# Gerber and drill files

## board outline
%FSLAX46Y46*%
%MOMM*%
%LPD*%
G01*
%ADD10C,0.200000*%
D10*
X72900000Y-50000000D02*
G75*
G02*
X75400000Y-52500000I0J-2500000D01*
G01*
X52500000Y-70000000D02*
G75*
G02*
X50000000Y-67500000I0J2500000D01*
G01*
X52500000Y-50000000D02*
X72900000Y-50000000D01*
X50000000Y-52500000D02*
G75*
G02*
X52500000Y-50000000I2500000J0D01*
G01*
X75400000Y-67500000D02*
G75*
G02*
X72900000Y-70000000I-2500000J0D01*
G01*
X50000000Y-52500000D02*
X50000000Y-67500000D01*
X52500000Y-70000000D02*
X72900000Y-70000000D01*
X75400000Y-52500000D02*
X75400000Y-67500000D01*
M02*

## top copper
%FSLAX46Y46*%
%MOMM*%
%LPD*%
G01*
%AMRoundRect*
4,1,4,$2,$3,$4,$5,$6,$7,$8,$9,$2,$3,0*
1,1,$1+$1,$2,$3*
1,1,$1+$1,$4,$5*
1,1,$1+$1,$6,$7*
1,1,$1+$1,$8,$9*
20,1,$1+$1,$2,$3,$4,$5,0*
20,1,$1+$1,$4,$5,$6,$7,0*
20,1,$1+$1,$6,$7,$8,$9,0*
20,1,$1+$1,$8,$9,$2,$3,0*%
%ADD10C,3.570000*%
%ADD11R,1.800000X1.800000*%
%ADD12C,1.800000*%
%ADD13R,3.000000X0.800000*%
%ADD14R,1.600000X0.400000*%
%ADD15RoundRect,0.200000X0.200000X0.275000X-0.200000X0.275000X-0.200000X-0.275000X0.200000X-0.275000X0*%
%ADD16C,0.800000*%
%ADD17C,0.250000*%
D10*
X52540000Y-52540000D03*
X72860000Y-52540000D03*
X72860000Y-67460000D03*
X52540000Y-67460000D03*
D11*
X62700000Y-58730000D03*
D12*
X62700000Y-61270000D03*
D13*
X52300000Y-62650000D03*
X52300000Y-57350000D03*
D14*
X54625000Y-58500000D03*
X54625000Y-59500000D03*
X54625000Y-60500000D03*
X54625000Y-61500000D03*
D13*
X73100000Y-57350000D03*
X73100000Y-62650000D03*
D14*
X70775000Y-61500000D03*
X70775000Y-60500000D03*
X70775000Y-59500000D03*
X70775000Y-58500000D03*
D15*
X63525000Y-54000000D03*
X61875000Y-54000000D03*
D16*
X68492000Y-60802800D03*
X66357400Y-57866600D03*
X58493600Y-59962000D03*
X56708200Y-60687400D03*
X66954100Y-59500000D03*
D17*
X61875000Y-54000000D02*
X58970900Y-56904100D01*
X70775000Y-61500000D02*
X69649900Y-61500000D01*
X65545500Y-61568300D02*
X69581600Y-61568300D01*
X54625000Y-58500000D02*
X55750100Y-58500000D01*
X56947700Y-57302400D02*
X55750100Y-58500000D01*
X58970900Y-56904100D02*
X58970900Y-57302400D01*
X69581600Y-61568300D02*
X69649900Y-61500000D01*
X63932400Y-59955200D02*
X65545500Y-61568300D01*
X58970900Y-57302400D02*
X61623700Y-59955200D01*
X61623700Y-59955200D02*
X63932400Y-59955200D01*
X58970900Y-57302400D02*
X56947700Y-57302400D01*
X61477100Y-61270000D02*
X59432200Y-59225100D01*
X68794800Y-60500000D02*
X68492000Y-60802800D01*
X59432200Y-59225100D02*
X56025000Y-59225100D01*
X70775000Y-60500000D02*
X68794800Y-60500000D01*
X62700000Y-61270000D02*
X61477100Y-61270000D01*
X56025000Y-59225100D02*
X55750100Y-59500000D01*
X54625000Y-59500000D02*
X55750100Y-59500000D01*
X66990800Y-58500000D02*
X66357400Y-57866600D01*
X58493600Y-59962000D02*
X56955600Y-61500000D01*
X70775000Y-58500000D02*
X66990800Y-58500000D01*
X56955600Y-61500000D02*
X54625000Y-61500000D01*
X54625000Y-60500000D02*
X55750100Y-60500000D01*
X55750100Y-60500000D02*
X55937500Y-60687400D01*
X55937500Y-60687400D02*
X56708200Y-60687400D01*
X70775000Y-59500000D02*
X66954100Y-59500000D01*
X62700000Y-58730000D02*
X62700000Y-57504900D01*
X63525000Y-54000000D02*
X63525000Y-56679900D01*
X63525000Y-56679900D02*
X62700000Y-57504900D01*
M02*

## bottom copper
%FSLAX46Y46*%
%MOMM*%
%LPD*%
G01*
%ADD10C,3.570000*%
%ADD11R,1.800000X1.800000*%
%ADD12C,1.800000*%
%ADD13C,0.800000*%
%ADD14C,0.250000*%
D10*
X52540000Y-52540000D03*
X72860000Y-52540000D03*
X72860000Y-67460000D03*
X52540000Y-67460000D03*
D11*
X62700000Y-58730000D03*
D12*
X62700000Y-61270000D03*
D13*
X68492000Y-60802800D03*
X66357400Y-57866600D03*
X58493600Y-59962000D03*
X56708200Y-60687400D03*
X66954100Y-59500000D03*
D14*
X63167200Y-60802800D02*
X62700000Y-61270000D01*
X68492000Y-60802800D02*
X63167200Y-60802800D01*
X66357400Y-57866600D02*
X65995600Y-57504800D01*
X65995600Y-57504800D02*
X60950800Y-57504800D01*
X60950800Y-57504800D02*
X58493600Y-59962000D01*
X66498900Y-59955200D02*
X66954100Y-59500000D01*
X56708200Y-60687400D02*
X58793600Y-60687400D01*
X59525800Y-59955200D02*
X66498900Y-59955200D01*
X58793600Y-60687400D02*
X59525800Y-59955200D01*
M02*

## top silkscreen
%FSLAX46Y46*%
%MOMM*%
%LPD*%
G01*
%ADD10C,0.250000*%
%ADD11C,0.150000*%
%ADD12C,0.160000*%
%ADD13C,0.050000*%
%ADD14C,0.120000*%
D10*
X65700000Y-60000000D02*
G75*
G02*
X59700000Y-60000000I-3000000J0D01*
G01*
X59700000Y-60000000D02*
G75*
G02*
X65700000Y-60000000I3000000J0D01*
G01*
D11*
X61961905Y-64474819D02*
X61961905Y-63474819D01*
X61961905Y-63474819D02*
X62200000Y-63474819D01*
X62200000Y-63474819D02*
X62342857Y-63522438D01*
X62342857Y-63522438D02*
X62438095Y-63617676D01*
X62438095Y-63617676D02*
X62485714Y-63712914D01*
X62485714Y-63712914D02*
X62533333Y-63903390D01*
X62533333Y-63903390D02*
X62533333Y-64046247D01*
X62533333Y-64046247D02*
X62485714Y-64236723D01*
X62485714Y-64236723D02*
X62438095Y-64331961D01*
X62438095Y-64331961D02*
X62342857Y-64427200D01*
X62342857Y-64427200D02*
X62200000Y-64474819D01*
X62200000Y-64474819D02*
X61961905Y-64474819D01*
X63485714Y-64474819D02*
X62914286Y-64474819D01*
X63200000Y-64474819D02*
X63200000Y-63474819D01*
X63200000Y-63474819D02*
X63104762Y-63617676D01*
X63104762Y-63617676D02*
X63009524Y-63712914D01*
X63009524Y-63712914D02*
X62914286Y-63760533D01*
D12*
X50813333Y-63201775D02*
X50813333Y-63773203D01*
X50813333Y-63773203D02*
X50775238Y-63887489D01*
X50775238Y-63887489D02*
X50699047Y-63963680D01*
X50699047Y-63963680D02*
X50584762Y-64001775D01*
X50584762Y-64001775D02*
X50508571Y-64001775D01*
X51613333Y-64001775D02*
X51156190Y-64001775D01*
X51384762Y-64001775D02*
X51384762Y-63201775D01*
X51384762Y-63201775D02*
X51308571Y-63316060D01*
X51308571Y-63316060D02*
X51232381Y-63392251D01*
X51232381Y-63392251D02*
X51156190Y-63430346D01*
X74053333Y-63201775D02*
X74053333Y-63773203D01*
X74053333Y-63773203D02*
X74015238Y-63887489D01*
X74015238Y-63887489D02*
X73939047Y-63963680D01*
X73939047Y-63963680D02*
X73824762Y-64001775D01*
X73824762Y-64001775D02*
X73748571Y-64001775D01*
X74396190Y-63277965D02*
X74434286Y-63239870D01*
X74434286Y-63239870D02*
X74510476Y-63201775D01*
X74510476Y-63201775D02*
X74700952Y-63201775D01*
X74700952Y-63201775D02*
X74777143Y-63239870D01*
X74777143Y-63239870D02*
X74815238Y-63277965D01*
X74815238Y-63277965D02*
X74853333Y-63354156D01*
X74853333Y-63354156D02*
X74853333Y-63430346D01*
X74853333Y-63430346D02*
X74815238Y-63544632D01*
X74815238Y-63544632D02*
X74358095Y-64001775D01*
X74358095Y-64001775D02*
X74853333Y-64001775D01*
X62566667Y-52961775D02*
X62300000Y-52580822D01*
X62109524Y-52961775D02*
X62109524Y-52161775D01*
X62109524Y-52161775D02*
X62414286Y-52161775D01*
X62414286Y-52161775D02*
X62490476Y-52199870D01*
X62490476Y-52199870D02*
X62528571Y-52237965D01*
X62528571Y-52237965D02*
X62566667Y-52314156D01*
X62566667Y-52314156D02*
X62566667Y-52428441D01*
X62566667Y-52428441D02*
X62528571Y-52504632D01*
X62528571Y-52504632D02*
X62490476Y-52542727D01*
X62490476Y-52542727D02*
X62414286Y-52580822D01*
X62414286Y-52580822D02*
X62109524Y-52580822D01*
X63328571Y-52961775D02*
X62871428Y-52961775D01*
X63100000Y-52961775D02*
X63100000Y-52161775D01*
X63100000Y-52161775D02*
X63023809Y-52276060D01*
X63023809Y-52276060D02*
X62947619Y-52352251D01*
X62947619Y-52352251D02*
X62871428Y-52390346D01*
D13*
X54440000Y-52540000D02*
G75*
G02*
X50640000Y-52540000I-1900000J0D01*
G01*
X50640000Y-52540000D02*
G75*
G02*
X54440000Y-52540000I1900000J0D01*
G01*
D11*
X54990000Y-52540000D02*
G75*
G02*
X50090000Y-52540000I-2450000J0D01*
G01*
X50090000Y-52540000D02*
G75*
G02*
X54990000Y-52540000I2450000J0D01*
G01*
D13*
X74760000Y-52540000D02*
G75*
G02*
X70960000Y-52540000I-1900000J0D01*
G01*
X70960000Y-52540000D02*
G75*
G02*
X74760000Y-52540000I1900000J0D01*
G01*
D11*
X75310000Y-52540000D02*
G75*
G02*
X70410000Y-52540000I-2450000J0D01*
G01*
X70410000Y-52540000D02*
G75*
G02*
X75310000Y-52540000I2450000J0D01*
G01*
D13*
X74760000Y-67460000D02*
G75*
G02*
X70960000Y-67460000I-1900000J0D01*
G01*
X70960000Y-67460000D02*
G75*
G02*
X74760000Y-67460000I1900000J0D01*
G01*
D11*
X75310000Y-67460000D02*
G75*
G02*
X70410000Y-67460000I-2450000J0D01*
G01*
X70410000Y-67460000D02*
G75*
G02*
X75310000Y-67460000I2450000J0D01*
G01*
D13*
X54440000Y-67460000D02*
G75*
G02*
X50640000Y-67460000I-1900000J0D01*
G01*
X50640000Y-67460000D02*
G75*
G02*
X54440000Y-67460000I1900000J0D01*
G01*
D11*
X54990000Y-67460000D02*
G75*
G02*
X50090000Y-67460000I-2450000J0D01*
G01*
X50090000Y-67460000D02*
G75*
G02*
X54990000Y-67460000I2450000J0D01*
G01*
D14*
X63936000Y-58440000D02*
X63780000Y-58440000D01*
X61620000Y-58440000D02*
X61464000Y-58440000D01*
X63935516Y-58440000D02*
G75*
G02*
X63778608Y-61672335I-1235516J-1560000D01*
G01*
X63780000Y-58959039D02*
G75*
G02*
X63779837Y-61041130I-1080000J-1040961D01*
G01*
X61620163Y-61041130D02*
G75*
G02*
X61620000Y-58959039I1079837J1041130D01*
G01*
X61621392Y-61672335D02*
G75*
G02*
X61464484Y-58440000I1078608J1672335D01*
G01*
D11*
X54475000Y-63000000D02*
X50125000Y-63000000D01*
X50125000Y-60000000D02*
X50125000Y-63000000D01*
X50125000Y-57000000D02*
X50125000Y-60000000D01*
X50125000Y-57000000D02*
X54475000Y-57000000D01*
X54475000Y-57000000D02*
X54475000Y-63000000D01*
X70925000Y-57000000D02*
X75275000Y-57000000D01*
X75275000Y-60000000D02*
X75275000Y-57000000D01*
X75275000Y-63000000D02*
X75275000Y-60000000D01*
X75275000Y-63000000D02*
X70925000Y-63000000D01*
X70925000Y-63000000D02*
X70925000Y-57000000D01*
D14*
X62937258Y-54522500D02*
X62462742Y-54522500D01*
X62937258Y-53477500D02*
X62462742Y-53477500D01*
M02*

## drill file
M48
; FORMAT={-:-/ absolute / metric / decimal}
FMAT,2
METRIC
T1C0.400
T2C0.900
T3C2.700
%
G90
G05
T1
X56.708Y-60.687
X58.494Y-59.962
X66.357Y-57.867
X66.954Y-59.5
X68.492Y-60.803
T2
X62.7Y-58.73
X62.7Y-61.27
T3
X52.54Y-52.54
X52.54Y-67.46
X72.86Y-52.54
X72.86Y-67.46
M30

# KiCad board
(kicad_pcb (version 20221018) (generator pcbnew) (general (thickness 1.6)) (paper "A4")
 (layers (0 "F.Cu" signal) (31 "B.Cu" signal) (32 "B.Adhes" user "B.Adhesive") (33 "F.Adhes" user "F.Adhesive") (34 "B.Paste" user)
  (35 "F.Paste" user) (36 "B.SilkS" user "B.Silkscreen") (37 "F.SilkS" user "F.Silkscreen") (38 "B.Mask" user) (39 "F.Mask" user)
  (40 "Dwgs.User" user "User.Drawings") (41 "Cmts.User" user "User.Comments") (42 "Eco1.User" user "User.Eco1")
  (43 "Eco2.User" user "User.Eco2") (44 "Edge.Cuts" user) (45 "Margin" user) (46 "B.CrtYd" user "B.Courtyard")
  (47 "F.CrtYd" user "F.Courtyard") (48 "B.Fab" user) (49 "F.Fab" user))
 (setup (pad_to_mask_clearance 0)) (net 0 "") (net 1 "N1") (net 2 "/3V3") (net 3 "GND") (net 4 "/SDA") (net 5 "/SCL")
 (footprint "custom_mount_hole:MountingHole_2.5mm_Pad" (layer "F.Cu") (at 52.54 52.54)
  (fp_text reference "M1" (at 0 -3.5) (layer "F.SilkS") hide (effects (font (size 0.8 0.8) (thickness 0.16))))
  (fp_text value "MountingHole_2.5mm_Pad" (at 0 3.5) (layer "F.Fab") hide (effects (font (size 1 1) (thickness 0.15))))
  (fp_circle (center 0 0) (end 1.9 0) (stroke (width 0.05) (type solid)) (fill none) (layer "F.SilkS"))
  (fp_circle (center 0 0) (end 2.45 0) (stroke (width 0.15) (type solid)) (fill none) (layer "F.SilkS"))
  (pad "~" thru_hole circle (at 0 0) (size 3.57 3.57) (drill 2.7) (layers "*.Cu" "*.Mask")))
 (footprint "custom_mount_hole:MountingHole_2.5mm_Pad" (layer "F.Cu") (at 72.86 52.54)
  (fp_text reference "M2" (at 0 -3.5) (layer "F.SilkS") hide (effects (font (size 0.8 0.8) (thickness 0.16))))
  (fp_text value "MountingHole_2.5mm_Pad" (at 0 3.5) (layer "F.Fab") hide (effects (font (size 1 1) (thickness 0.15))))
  (fp_circle (center 0 0) (end 1.9 0) (stroke (width 0.05) (type solid)) (fill none) (layer "F.SilkS"))
  (fp_circle (center 0 0) (end 2.45 0) (stroke (width 0.15) (type solid)) (fill none) (layer "F.SilkS"))
  (pad "~" thru_hole circle (at 0 0) (size 3.57 3.57) (drill 2.7) (layers "*.Cu" "*.Mask")))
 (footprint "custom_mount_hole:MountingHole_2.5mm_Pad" (layer "F.Cu") (at 72.86 67.46)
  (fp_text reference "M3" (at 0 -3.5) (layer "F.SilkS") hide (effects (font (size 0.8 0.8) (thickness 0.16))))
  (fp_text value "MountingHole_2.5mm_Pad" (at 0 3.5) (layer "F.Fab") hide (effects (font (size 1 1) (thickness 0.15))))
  (fp_circle (center 0 0) (end 1.9 0) (stroke (width 0.05) (type solid)) (fill none) (layer "F.SilkS"))
  (fp_circle (center 0 0) (end 2.45 0) (stroke (width 0.15) (type solid)) (fill none) (layer "F.SilkS"))
  (pad "~" thru_hole circle (at 0 0) (size 3.57 3.57) (drill 2.7) (layers "*.Cu" "*.Mask")))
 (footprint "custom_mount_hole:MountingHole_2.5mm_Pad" (layer "F.Cu") (at 52.54 67.46)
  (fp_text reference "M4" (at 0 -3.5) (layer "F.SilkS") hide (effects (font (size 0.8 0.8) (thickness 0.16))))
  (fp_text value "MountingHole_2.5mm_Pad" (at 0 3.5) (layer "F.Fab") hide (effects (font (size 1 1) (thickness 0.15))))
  (fp_circle (center 0 0) (end 1.9 0) (stroke (width 0.05) (type solid)) (fill none) (layer "F.SilkS"))
  (fp_circle (center 0 0) (end 2.45 0) (stroke (width 0.15) (type solid)) (fill none) (layer "F.SilkS"))
  (pad "~" thru_hole circle (at 0 0) (size 3.57 3.57) (drill 2.7) (layers "*.Cu" "*.Mask")))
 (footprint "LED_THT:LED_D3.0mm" (layer "F.Cu") (at 62.7 58.73 -90)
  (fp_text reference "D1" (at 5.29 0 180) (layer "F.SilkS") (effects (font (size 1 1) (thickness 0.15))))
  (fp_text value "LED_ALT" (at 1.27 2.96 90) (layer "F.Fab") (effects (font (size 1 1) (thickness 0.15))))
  (fp_line (start -0.29 -1.236) (end -0.29 -1.08) (stroke (width 0.12) (type solid)) (layer "F.SilkS"))
  (fp_line (start -0.29 1.08) (end -0.29 1.236) (stroke (width 0.12) (type solid)) (layer "F.SilkS"))
  (fp_arc (start -0.29 -1.235516) (mid 1.366487 -1.987659) (end 2.942335 -1.078608) (stroke (width 0.12) (type solid)) (layer "F.SilkS"))
  (fp_arc (start 0.229039 -1.08) (mid 1.270117 -1.5) (end 2.31113 -1.079837) (stroke (width 0.12) (type solid)) (layer "F.SilkS"))
  (fp_arc (start 2.31113 1.079837) (mid 1.270117 1.5) (end 0.229039 1.08) (stroke (width 0.12) (type solid)) (layer "F.SilkS"))
  (fp_arc (start 2.942335 1.078608) (mid 1.366487 1.987659) (end -0.29 1.235516) (stroke (width 0.12) (type solid)) (layer "F.SilkS"))
  (pad "1" thru_hole rect (at 0 0 270) (size 1.8 1.8) (drill 0.9) (layers "*.Cu" "*.Mask") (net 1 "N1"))
  (pad "2" thru_hole circle (at 2.54 0 270) (size 1.8 1.8) (drill 0.9) (layers "*.Cu" "*.Mask") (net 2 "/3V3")))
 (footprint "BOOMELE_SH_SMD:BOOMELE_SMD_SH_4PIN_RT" (layer "F.Cu") (at 52.78 60 90)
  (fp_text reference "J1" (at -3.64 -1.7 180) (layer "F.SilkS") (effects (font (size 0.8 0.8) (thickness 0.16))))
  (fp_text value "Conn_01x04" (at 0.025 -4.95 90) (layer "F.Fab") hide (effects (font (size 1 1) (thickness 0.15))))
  (fp_line (start -3 1.695) (end -3 -2.655) (stroke (width 0.15) (type solid)) (layer "F.SilkS"))
  (fp_line (start 0 -2.655) (end -3 -2.655) (stroke (width 0.15) (type solid)) (layer "F.SilkS"))
  (fp_line (start 3 -2.655) (end 0 -2.655) (stroke (width 0.15) (type solid)) (layer "F.SilkS"))
  (fp_line (start 3 -2.655) (end 3 1.695) (stroke (width 0.15) (type solid)) (layer "F.SilkS"))
  (fp_line (start 3 1.695) (end -3 1.695) (stroke (width 0.15) (type solid)) (layer "F.SilkS"))
  (pad "" smd rect (at -2.65 -0.48 270) (size 0.8 3) (layers "F.Cu" "F.Paste" "F.Mask"))
  (pad "" smd rect (at 2.65 -0.48 270) (size 0.8 3) (layers "F.Cu" "F.Paste" "F.Mask"))
  (pad "1" smd rect (at 1.5 1.845 270) (size 0.4 1.6) (layers "F.Cu" "F.Paste" "F.Mask") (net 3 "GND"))
  (pad "2" smd rect (at 0.5 1.845 270) (size 0.4 1.6) (layers "F.Cu" "F.Paste" "F.Mask") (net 2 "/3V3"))
  (pad "3" smd rect (at -0.5 1.845 270) (size 0.4 1.6) (layers "F.Cu" "F.Paste" "F.Mask") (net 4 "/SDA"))
  (pad "4" smd rect (at -1.5 1.845 270) (size 0.4 1.6) (layers "F.Cu" "F.Paste" "F.Mask") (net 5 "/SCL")))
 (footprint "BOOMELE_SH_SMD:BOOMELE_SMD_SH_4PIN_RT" (layer "F.Cu") (at 72.62 60 -90)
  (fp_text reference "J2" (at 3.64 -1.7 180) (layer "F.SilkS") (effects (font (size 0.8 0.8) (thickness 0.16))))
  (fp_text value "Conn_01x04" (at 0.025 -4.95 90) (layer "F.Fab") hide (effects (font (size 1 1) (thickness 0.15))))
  (fp_line (start -3 1.695) (end -3 -2.655) (stroke (width 0.15) (type solid)) (layer "F.SilkS"))
  (fp_line (start 0 -2.655) (end -3 -2.655) (stroke (width 0.15) (type solid)) (layer "F.SilkS"))
  (fp_line (start 3 -2.655) (end 0 -2.655) (stroke (width 0.15) (type solid)) (layer "F.SilkS"))
  (fp_line (start 3 -2.655) (end 3 1.695) (stroke (width 0.15) (type solid)) (layer "F.SilkS"))
  (fp_line (start 3 1.695) (end -3 1.695) (stroke (width 0.15) (type solid)) (layer "F.SilkS"))
  (pad "" smd rect (at -2.65 -0.48 90) (size 0.8 3) (layers "F.Cu" "F.Paste" "F.Mask"))
  (pad "" smd rect (at 2.65 -0.48 90) (size 0.8 3) (layers "F.Cu" "F.Paste" "F.Mask"))
  (pad "1" smd rect (at 1.5 1.845 90) (size 0.4 1.6) (layers "F.Cu" "F.Paste" "F.Mask") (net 3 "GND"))
  (pad "2" smd rect (at 0.5 1.845 90) (size 0.4 1.6) (layers "F.Cu" "F.Paste" "F.Mask") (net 2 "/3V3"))
  (pad "3" smd rect (at -0.5 1.845 90) (size 0.4 1.6) (layers "F.Cu" "F.Paste" "F.Mask") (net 4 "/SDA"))
  (pad "4" smd rect (at -1.5 1.845 90) (size 0.4 1.6) (layers "F.Cu" "F.Paste" "F.Mask") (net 5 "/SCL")))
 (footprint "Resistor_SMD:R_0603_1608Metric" (layer "F.Cu") (at 62.7 54 180)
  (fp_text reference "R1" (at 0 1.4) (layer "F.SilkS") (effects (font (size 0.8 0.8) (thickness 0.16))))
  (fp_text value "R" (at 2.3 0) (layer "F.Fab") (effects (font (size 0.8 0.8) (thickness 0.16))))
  (fp_line (start -0.237258 -0.5225) (end 0.237258 -0.5225) (stroke (width 0.12) (type solid)) (layer "F.SilkS"))
  (fp_line (start -0.237258 0.5225) (end 0.237258 0.5225) (stroke (width 0.12) (type solid)) (layer "F.SilkS"))
  (pad "1" smd roundrect (at -0.825 0 180) (size 0.8 0.95) (layers "F.Cu" "F.Paste" "F.Mask") (roundrect_rratio 0.25) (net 1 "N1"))
  (pad "2" smd roundrect (at 0.825 0 180) (size 0.8 0.95) (layers "F.Cu" "F.Paste" "F.Mask") (roundrect_rratio 0.25) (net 3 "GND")))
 (gr_circle (center 62.7 60) (end 65.7 60) (stroke (width 0.25) (type solid)) (fill none) (layer "F.SilkS"))
 (gr_arc (start 72.9 50) (mid 74.667767 50.732233) (end 75.4 52.5) (stroke (width 0.2) (type solid)) (layer "Edge.Cuts"))
 (gr_arc (start 52.5 70) (mid 50.732233 69.267767) (end 50 67.5) (stroke (width 0.2) (type solid)) (layer "Edge.Cuts"))
 (gr_line (start 52.5 50) (end 72.9 50) (stroke (width 0.2) (type solid)) (layer "Edge.Cuts"))
 (gr_arc (start 50 52.5) (mid 50.732233 50.732233) (end 52.5 50) (stroke (width 0.2) (type solid)) (layer "Edge.Cuts"))
 (gr_arc (start 75.4 67.5) (mid 74.667767 69.267767) (end 72.9 70) (stroke (width 0.2) (type solid)) (layer "Edge.Cuts"))
 (gr_line (start 50 52.5) (end 50 67.5) (stroke (width 0.2) (type solid)) (layer "Edge.Cuts"))
 (gr_line (start 52.5 70) (end 72.9 70) (stroke (width 0.2) (type solid)) (layer "Edge.Cuts"))
 (gr_line (start 75.4 52.5) (end 75.4 67.5) (stroke (width 0.2) (type solid)) (layer "Edge.Cuts"))
 (segment (start 61.875 54) (end 58.9709 56.9041) (width 0.25) (layer "F.Cu") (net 3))
 (segment (start 70.775 61.5) (end 69.6499 61.5) (width 0.25) (layer "F.Cu") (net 3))
 (segment (start 65.5455 61.5683) (end 69.5816 61.5683) (width 0.25) (layer "F.Cu") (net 3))
 (segment (start 54.625 58.5) (end 55.7501 58.5) (width 0.25) (layer "F.Cu") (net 3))
 (segment (start 56.9477 57.3024) (end 55.7501 58.5) (width 0.25) (layer "F.Cu") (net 3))
 (segment (start 58.9709 56.9041) (end 58.9709 57.3024) (width 0.25) (layer "F.Cu") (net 3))
 (segment (start 69.5816 61.5683) (end 69.6499 61.5) (width 0.25) (layer "F.Cu") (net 3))
 (segment (start 63.9324 59.9552) (end 65.5455 61.5683) (width 0.25) (layer "F.Cu") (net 3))
 (segment (start 58.9709 57.3024) (end 61.6237 59.9552) (width 0.25) (layer "F.Cu") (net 3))
 (segment (start 61.6237 59.9552) (end 63.9324 59.9552) (width 0.25) (layer "F.Cu") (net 3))
 (segment (start 58.9709 57.3024) (end 56.9477 57.3024) (width 0.25) (layer "F.Cu") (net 3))
 (segment (start 61.4771 61.27) (end 59.4322 59.2251) (width 0.25) (layer "F.Cu") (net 2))
 (segment (start 68.7948 60.5) (end 68.492 60.8028) (width 0.25) (layer "F.Cu") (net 2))
 (segment (start 59.4322 59.2251) (end 56.025 59.2251) (width 0.25) (layer "F.Cu") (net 2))
 (segment (start 70.775 60.5) (end 68.7948 60.5) (width 0.25) (layer "F.Cu") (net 2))
 (segment (start 62.7 61.27) (end 61.4771 61.27) (width 0.25) (layer "F.Cu") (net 2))
 (segment (start 56.025 59.2251) (end 55.7501 59.5) (width 0.25) (layer "F.Cu") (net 2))
 (segment (start 54.625 59.5) (end 55.7501 59.5) (width 0.25) (layer "F.Cu") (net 2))
 (via (at 68.492 60.8028) (size 0.8) (drill 0.4) (layers "F.Cu" "B.Cu") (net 2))
 (segment (start 63.1672 60.8028) (end 62.7 61.27) (width 0.25) (layer "B.Cu") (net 2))
 (segment (start 68.492 60.8028) (end 63.1672 60.8028) (width 0.25) (layer "B.Cu") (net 2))
 (segment (start 66.9908 58.5) (end 66.3574 57.8666) (width 0.25) (layer "F.Cu") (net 5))
 (segment (start 58.4936 59.962) (end 56.9556 61.5) (width 0.25) (layer "F.Cu") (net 5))
 (segment (start 70.775 58.5) (end 66.9908 58.5) (width 0.25) (layer "F.Cu") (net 5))
 (segment (start 56.9556 61.5) (end 54.625 61.5) (width 0.25) (layer "F.Cu") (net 5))
 (via (at 66.3574 57.8666) (size 0.8) (drill 0.4) (layers "F.Cu" "B.Cu") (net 5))
 (via (at 58.4936 59.962) (size 0.8) (drill 0.4) (layers "F.Cu" "B.Cu") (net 5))
 (segment (start 66.3574 57.8666) (end 65.9956 57.5048) (width 0.25) (layer "B.Cu") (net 5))
 (segment (start 65.9956 57.5048) (end 60.9508 57.5048) (width 0.25) (layer "B.Cu") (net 5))
 (segment (start 60.9508 57.5048) (end 58.4936 59.962) (width 0.25) (layer "B.Cu") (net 5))
 (segment (start 54.625 60.5) (end 55.7501 60.5) (width 0.25) (layer "F.Cu") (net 4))
 (segment (start 55.7501 60.5) (end 55.9375 60.6874) (width 0.25) (layer "F.Cu") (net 4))
 (segment (start 55.9375 60.6874) (end 56.7082 60.6874) (width 0.25) (layer "F.Cu") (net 4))
 (segment (start 70.775 59.5) (end 66.9541 59.5) (width 0.25) (layer "F.Cu") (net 4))
 (via (at 56.7082 60.6874) (size 0.8) (drill 0.4) (layers "F.Cu" "B.Cu") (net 4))
 (via (at 66.9541 59.5) (size 0.8) (drill 0.4) (layers "F.Cu" "B.Cu") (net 4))
 (segment (start 66.4989 59.9552) (end 66.9541 59.5) (width 0.25) (layer "B.Cu") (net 4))
 (segment (start 56.7082 60.6874) (end 58.7936 60.6874) (width 0.25) (layer "B.Cu") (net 4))
 (segment (start 59.5258 59.9552) (end 66.4989 59.9552) (width 0.25) (layer "B.Cu") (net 4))
 (segment (start 58.7936 60.6874) (end 59.5258 59.9552) (width 0.25) (layer "B.Cu") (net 4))
 (segment (start 62.7 58.73) (end 62.7 57.5049) (width 0.25) (layer "F.Cu") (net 1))
 (segment (start 63.525 54) (end 63.525 56.6799) (width 0.25) (layer "F.Cu") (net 1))
 (segment (start 63.525 56.6799) (end 62.7 57.5049) (width 0.25) (layer "F.Cu") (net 1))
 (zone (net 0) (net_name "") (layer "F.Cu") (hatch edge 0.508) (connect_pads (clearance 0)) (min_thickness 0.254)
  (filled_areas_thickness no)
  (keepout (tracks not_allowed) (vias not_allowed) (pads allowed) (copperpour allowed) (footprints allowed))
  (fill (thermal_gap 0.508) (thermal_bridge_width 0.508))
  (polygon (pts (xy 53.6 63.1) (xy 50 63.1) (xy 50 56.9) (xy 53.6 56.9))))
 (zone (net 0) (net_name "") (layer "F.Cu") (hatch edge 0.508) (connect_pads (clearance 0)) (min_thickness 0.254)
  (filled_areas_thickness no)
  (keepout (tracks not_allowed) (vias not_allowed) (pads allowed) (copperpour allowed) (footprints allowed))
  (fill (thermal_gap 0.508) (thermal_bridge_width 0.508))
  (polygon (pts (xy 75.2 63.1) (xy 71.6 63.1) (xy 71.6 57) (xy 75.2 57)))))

